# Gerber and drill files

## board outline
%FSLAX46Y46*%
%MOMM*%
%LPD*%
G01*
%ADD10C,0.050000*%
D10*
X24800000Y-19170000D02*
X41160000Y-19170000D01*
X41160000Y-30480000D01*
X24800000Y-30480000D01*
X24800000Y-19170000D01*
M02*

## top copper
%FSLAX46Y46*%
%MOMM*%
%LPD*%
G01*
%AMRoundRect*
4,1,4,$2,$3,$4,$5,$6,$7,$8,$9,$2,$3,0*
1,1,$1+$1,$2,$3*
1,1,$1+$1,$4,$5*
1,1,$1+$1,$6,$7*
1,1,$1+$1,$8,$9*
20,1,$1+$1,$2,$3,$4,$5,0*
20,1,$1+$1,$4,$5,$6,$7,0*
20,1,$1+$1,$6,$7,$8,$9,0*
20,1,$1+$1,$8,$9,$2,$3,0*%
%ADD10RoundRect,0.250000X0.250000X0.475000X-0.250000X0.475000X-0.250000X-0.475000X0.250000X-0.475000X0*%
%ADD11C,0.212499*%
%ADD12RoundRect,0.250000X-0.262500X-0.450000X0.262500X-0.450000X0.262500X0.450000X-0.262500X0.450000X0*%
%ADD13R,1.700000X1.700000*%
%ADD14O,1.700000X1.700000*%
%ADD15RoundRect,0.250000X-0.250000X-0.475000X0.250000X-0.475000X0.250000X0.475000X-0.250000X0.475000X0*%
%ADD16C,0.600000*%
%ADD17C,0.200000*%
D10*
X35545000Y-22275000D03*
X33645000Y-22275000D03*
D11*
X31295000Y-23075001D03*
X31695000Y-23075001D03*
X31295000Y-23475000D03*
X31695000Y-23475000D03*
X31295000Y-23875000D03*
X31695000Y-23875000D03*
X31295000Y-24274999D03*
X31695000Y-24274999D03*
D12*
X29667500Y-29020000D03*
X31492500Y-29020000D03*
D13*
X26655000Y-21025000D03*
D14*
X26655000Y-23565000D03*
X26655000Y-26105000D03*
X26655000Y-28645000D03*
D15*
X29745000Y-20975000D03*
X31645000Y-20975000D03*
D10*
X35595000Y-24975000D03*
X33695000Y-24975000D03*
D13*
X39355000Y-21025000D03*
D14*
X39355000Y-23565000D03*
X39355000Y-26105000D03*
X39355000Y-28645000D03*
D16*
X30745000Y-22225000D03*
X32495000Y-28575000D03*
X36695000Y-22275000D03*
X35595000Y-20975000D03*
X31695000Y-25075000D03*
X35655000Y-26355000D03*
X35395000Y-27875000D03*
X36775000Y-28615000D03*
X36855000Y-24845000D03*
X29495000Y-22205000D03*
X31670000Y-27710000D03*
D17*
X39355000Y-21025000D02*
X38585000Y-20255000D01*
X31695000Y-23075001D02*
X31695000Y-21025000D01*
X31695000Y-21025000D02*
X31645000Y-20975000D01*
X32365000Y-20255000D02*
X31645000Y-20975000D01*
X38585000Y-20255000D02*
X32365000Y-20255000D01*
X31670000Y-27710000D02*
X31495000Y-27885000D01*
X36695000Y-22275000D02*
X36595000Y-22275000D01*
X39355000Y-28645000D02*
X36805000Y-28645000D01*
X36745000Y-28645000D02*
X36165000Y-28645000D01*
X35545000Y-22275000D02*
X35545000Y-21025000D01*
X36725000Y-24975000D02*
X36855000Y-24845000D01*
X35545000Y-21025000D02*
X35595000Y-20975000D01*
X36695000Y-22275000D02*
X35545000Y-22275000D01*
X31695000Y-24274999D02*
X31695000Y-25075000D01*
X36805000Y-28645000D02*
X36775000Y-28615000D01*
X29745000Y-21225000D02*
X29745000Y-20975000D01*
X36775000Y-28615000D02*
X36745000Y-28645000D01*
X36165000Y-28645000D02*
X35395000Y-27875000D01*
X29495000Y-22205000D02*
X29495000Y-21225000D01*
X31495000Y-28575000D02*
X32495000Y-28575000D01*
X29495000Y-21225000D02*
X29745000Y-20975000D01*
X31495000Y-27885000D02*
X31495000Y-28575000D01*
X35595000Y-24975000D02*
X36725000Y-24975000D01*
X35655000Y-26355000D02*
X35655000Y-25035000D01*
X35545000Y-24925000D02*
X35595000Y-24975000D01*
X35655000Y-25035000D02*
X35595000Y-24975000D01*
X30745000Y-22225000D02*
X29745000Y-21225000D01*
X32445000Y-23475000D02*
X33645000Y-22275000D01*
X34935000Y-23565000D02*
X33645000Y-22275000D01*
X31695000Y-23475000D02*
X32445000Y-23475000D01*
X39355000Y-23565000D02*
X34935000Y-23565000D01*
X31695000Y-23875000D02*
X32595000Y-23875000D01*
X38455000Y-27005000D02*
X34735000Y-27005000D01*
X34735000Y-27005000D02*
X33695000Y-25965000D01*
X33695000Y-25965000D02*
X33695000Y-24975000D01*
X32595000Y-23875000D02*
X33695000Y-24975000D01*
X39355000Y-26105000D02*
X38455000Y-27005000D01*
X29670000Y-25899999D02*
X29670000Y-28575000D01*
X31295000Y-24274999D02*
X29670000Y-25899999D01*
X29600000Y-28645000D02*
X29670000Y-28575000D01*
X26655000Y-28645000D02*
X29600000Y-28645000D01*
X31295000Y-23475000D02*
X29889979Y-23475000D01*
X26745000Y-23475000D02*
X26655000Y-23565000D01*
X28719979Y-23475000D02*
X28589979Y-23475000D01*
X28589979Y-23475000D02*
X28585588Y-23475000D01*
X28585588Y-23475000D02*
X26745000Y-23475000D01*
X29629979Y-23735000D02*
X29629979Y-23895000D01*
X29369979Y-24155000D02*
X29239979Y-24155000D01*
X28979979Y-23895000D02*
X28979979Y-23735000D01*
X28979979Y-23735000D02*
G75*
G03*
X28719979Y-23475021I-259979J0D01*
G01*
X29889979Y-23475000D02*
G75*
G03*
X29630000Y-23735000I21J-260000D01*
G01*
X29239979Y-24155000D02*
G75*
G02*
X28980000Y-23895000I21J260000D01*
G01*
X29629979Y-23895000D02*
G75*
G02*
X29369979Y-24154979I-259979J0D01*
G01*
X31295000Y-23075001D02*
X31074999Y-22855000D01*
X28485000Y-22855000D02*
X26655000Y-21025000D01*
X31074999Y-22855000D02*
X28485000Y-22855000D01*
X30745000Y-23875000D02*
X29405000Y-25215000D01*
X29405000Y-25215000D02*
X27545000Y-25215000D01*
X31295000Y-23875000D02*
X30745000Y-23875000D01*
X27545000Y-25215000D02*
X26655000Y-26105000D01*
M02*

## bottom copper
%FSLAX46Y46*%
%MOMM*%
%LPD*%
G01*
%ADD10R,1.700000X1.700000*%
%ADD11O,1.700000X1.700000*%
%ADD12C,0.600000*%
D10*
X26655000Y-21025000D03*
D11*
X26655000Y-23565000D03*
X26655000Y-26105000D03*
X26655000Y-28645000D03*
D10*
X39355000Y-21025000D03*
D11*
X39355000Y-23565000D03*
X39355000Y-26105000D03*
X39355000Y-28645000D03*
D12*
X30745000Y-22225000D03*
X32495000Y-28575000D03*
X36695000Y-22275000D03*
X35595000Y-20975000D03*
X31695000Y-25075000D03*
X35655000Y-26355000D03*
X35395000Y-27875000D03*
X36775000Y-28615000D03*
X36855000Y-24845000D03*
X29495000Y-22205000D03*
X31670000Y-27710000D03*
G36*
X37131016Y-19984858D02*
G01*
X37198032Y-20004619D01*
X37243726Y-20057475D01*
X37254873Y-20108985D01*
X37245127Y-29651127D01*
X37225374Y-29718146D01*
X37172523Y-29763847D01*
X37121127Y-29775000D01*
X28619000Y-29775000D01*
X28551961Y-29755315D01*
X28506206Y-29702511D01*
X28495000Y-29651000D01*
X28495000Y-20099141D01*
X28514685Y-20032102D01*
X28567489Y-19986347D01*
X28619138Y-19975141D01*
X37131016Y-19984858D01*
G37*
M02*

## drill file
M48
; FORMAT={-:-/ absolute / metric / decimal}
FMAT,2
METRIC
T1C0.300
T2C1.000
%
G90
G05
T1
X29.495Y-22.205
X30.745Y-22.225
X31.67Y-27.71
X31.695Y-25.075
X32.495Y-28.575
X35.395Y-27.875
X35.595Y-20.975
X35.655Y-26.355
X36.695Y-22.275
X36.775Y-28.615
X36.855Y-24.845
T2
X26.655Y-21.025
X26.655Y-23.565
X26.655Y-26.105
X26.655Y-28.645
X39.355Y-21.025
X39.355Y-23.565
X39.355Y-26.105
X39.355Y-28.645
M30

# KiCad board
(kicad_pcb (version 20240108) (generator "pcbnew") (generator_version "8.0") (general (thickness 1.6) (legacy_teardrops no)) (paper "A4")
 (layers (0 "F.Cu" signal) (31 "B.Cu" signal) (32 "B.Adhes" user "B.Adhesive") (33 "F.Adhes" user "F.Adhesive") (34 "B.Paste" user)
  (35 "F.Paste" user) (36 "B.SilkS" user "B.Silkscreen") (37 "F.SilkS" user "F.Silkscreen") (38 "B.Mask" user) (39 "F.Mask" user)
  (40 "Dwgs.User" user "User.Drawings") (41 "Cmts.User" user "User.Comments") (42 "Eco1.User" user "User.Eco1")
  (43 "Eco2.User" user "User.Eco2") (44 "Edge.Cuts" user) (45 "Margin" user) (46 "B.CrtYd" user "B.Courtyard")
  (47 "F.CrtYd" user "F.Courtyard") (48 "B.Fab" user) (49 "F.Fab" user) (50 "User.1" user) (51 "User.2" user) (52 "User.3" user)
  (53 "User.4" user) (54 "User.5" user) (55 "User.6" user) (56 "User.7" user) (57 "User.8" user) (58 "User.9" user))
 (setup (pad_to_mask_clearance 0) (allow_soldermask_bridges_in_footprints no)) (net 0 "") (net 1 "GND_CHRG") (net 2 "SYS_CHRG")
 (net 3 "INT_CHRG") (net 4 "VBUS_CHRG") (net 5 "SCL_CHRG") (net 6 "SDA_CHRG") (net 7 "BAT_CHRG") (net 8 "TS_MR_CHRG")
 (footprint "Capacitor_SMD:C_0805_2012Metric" (layer "F.Cu") (at 34.595 22.275 180)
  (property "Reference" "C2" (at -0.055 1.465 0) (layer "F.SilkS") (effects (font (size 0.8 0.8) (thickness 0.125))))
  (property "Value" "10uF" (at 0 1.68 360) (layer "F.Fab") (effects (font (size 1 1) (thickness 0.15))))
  (pad "1" smd roundrect (at -0.95 0 180) (size 1 1.45) (layers "F.Cu" "F.Paste" "F.Mask") (roundrect_rratio 0.25) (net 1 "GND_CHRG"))
  (pad "2" smd roundrect (at 0.95 0 180) (size 1 1.45) (layers "F.Cu" "F.Paste" "F.Mask") (roundrect_rratio 0.25) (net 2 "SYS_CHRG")))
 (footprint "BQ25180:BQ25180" (layer "F.Cu") (at 31.495 23.675)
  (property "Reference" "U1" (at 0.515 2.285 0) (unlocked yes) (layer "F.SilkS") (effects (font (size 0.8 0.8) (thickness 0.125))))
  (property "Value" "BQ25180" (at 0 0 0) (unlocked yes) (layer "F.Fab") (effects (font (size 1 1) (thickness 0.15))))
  (pad "1" smd circle (at -0.2 -0.599999) (size 0.212499 0.212499) (layers "F.Cu" "F.Paste" "F.Mask") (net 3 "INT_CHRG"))
  (pad "2" smd circle (at 0.2 -0.599999) (size 0.212499 0.212499) (layers "F.Cu" "F.Paste" "F.Mask") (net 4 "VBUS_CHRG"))
  (pad "3" smd circle (at -0.2 -0.2) (size 0.212499 0.212499) (layers "F.Cu" "F.Paste" "F.Mask") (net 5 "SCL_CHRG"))
  (pad "4" smd circle (at 0.2 -0.2) (size 0.212499 0.212499) (layers "F.Cu" "F.Paste" "F.Mask") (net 2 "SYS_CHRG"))
  (pad "5" smd circle (at -0.2 0.2) (size 0.212499 0.212499) (layers "F.Cu" "F.Paste" "F.Mask") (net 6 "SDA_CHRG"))
  (pad "6" smd circle (at 0.2 0.2) (size 0.212499 0.212499) (layers "F.Cu" "F.Paste" "F.Mask") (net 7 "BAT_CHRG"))
  (pad "7" smd circle (at -0.2 0.599999) (size 0.212499 0.212499) (layers "F.Cu" "F.Paste" "F.Mask") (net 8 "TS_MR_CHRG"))
  (pad "8" smd circle (at 0.2 0.599999) (size 0.212499 0.212499) (layers "F.Cu" "F.Paste" "F.Mask") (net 1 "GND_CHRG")))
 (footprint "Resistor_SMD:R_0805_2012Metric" (layer "F.Cu") (at 30.58 29.02)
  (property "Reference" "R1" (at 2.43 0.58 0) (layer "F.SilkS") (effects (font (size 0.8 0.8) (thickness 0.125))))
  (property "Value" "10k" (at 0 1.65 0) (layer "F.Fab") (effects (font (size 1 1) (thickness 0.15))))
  (pad "1" smd roundrect (at -0.9125 0) (size 1.025 1.4) (layers "F.Cu" "F.Paste" "F.Mask") (roundrect_rratio 0.243902) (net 8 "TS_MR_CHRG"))
  (pad "2" smd roundrect (at 0.9125 0) (size 1.025 1.4) (layers "F.Cu" "F.Paste" "F.Mask") (roundrect_rratio 0.243902) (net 1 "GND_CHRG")))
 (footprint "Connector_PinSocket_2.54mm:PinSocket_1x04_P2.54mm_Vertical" (layer "F.Cu") (at 26.655 21.025)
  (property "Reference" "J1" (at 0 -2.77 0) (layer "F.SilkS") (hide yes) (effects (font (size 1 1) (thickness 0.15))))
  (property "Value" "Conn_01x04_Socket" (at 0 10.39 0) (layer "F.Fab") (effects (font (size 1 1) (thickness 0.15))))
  (pad "1" thru_hole rect (at 0 0) (size 1.7 1.7) (drill 1) (layers "*.Cu" "*.Mask") (remove_unused_layers no) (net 3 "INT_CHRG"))
  (pad "2" thru_hole oval (at 0 2.54) (size 1.7 1.7) (drill 1) (layers "*.Cu" "*.Mask") (remove_unused_layers no) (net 5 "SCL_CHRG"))
  (pad "3" thru_hole oval (at 0 5.08) (size 1.7 1.7) (drill 1) (layers "*.Cu" "*.Mask") (remove_unused_layers no) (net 6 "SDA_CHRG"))
  (pad "4" thru_hole oval (at 0 7.62) (size 1.7 1.7) (drill 1) (layers "*.Cu" "*.Mask") (remove_unused_layers no) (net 8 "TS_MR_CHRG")))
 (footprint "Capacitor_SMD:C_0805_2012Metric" (layer "F.Cu") (at 30.695 20.975)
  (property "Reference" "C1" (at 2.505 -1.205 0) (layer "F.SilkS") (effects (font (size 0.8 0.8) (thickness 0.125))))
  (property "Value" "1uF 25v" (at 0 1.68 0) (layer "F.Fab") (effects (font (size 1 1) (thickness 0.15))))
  (pad "1" smd roundrect (at -0.95 0) (size 1 1.45) (layers "F.Cu" "F.Paste" "F.Mask") (roundrect_rratio 0.25) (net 1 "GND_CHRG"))
  (pad "2" smd roundrect (at 0.95 0) (size 1 1.45) (layers "F.Cu" "F.Paste" "F.Mask") (roundrect_rratio 0.25) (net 4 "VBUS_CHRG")))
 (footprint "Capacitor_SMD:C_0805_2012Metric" (layer "F.Cu") (at 34.645 24.975 180)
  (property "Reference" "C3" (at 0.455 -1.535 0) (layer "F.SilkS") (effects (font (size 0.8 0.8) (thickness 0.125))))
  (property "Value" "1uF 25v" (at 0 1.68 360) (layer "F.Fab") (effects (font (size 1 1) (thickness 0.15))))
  (pad "1" smd roundrect (at -0.95 0 180) (size 1 1.45) (layers "F.Cu" "F.Paste" "F.Mask") (roundrect_rratio 0.25) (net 1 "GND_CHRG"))
  (pad "2" smd roundrect (at 0.95 0 180) (size 1 1.45) (layers "F.Cu" "F.Paste" "F.Mask") (roundrect_rratio 0.25) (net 7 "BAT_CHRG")))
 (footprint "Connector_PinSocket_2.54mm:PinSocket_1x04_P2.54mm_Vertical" (layer "F.Cu") (at 39.355 21.025)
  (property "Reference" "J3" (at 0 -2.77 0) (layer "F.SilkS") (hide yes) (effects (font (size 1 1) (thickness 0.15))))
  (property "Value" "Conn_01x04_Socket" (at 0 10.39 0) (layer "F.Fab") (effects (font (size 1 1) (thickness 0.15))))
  (pad "1" thru_hole rect (at 0 0) (size 1.7 1.7) (drill 1) (layers "*.Cu" "*.Mask") (remove_unused_layers no) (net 4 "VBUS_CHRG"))
  (pad "2" thru_hole oval (at 0 2.54) (size 1.7 1.7) (drill 1) (layers "*.Cu" "*.Mask") (remove_unused_layers no) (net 2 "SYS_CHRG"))
  (pad "3" thru_hole oval (at 0 5.08) (size 1.7 1.7) (drill 1) (layers "*.Cu" "*.Mask") (remove_unused_layers no) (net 7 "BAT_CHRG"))
  (pad "4" thru_hole oval (at 0 7.62) (size 1.7 1.7) (drill 1) (layers "*.Cu" "*.Mask") (remove_unused_layers no) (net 1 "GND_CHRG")))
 (gr_rect (start 24.8 19.17) (end 41.16 30.48) (stroke (width 0.05) (type default)) (fill none) (layer "Edge.Cuts"))
 (segment (start 39.355 21.025) (end 38.585 20.255) (width 0.2) (layer "F.Cu") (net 4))
 (segment (start 31.695 23.075001) (end 31.695 21.025) (width 0.2) (layer "F.Cu") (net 4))
 (segment (start 31.695 21.025) (end 31.645 20.975) (width 0.2) (layer "F.Cu") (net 4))
 (segment (start 32.365 20.255) (end 31.645 20.975) (width 0.2) (layer "F.Cu") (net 4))
 (segment (start 38.585 20.255) (end 32.365 20.255) (width 0.2) (layer "F.Cu") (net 4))
 (segment (start 31.67 27.71) (end 31.495 27.885) (width 0.2) (layer "F.Cu") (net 1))
 (segment (start 36.695 22.275) (end 36.595 22.275) (width 0.2) (layer "F.Cu") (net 1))
 (segment (start 39.355 28.645) (end 36.805 28.645) (width 0.2) (layer "F.Cu") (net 1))
 (segment (start 36.745 28.645) (end 36.165 28.645) (width 0.2) (layer "F.Cu") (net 1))
 (segment (start 35.545 22.275) (end 35.545 21.025) (width 0.2) (layer "F.Cu") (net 1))
 (segment (start 36.725 24.975) (end 36.855 24.845) (width 0.2) (layer "F.Cu") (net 1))
 (segment (start 35.545 21.025) (end 35.595 20.975) (width 0.2) (layer "F.Cu") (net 1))
 (segment (start 36.695 22.275) (end 35.545 22.275) (width 0.2) (layer "F.Cu") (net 1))
 (segment (start 31.695 24.274999) (end 31.695 25.075) (width 0.2) (layer "F.Cu") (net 1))
 (segment (start 36.805 28.645) (end 36.775 28.615) (width 0.2) (layer "F.Cu") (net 1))
 (segment (start 29.745 21.225) (end 29.745 20.975) (width 0.2) (layer "F.Cu") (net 1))
 (segment (start 36.775 28.615) (end 36.745 28.645) (width 0.2) (layer "F.Cu") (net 1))
 (segment (start 36.165 28.645) (end 35.395 27.875) (width 0.2) (layer "F.Cu") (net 1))
 (segment (start 29.495 22.205) (end 29.495 21.225) (width 0.2) (layer "F.Cu") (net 1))
 (segment (start 31.495 28.575) (end 32.495 28.575) (width 0.2) (layer "F.Cu") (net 1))
 (segment (start 29.495 21.225) (end 29.745 20.975) (width 0.2) (layer "F.Cu") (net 1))
 (segment (start 31.495 27.885) (end 31.495 28.575) (width 0.2) (layer "F.Cu") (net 1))
 (segment (start 35.595 24.975) (end 36.725 24.975) (width 0.2) (layer "F.Cu") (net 1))
 (segment (start 35.655 26.355) (end 35.655 25.035) (width 0.2) (layer "F.Cu") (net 1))
 (segment (start 35.545 24.925) (end 35.595 24.975) (width 0.2) (layer "F.Cu") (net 1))
 (segment (start 35.655 25.035) (end 35.595 24.975) (width 0.2) (layer "F.Cu") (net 1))
 (segment (start 30.745 22.225) (end 29.745 21.225) (width 0.2) (layer "F.Cu") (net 1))
 (via (at 30.745 22.225) (size 0.6) (drill 0.3) (layers "F.Cu" "B.Cu") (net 1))
 (via (at 32.495 28.575) (size 0.6) (drill 0.3) (layers "F.Cu" "B.Cu") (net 1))
 (via (at 36.695 22.275) (size 0.6) (drill 0.3) (layers "F.Cu" "B.Cu") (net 1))
 (via (at 35.595 20.975) (size 0.6) (drill 0.3) (layers "F.Cu" "B.Cu") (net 1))
 (via (at 31.695 25.075) (size 0.6) (drill 0.3) (layers "F.Cu" "B.Cu") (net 1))
 (via (at 35.655 26.355) (size 0.6) (drill 0.3) (layers "F.Cu" "B.Cu") (free yes) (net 1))
 (via (at 35.395 27.875) (size 0.6) (drill 0.3) (layers "F.Cu" "B.Cu") (free yes) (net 1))
 (via (at 36.775 28.615) (size 0.6) (drill 0.3) (layers "F.Cu" "B.Cu") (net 1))
 (via (at 36.855 24.845) (size 0.6) (drill 0.3) (layers "F.Cu" "B.Cu") (free yes) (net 1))
 (via (at 29.495 22.205) (size 0.6) (drill 0.3) (layers "F.Cu" "B.Cu") (free yes) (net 1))
 (via (at 31.67 27.71) (size 0.6) (drill 0.3) (layers "F.Cu" "B.Cu") (free yes) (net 1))
 (segment (start 32.445 23.475) (end 33.645 22.275) (width 0.2) (layer "F.Cu") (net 2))
 (segment (start 34.935 23.565) (end 33.645 22.275) (width 0.2) (layer "F.Cu") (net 2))
 (segment (start 31.695 23.475) (end 32.445 23.475) (width 0.2) (layer "F.Cu") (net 2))
 (segment (start 39.355 23.565) (end 34.935 23.565) (width 0.2) (layer "F.Cu") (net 2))
 (segment (start 31.695 23.875) (end 32.595 23.875) (width 0.2) (layer "F.Cu") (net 7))
 (segment (start 38.455 27.005) (end 34.735 27.005) (width 0.2) (layer "F.Cu") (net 7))
 (segment (start 34.735 27.005) (end 33.695 25.965) (width 0.2) (layer "F.Cu") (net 7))
 (segment (start 33.695 25.965) (end 33.695 24.975) (width 0.2) (layer "F.Cu") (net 7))
 (segment (start 32.595 23.875) (end 33.695 24.975) (width 0.2) (layer "F.Cu") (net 7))
 (segment (start 39.355 26.105) (end 38.455 27.005) (width 0.2) (layer "F.Cu") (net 7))
 (segment (start 29.67 25.899999) (end 29.67 28.575) (width 0.2) (layer "F.Cu") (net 8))
 (segment (start 31.295 24.274999) (end 29.67 25.899999) (width 0.2) (layer "F.Cu") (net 8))
 (segment (start 29.6 28.645) (end 29.67 28.575) (width 0.2) (layer "F.Cu") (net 8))
 (segment (start 26.655 28.645) (end 29.6 28.645) (width 0.2) (layer "F.Cu") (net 8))
 (segment (start 31.295 23.475) (end 29.889979 23.475) (width 0.2) (layer "F.Cu") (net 5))
 (segment (start 26.745 23.475) (end 26.655 23.565) (width 0.2) (layer "F.Cu") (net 5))
 (segment (start 28.719979 23.475) (end 28.589979 23.475) (width 0.2) (layer "F.Cu") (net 5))
 (segment (start 28.589979 23.475) (end 28.585588 23.475) (width 0.2) (layer "F.Cu") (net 5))
 (segment (start 28.585588 23.475) (end 26.745 23.475) (width 0.2) (layer "F.Cu") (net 5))
 (segment (start 29.629979 23.735) (end 29.629979 23.895) (width 0.2) (layer "F.Cu") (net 5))
 (segment (start 29.369979 24.155) (end 29.239979 24.155) (width 0.2) (layer "F.Cu") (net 5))
 (segment (start 28.979979 23.895) (end 28.979979 23.735) (width 0.2) (layer "F.Cu") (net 5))
 (arc (start 28.979979 23.735) (mid 28.903827 23.551152) (end 28.719979 23.475) (width 0.2) (layer "F.Cu") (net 5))
 (arc (start 29.889979 23.475) (mid 29.706131 23.551152) (end 29.629979 23.735) (width 0.2) (layer "F.Cu") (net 5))
 (arc (start 29.239979 24.155) (mid 29.056131 24.078848) (end 28.979979 23.895) (width 0.2) (layer "F.Cu") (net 5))
 (arc (start 29.629979 23.895) (mid 29.553827 24.078848) (end 29.369979 24.155) (width 0.2) (layer "F.Cu") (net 5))
 (segment (start 31.295 23.075001) (end 31.074999 22.855) (width 0.2) (layer "F.Cu") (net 3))
 (segment (start 28.485 22.855) (end 26.655 21.025) (width 0.2) (layer "F.Cu") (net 3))
 (segment (start 31.074999 22.855) (end 28.485 22.855) (width 0.2) (layer "F.Cu") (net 3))
 (segment (start 30.745 23.875) (end 29.405 25.215) (width 0.2) (layer "F.Cu") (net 6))
 (segment (start 29.405 25.215) (end 27.545 25.215) (width 0.2) (layer "F.Cu") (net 6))
 (segment (start 31.295 23.875) (end 30.745 23.875) (width 0.2) (layer "F.Cu") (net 6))
 (segment (start 27.545 25.215) (end 26.655 26.105) (width 0.2) (layer "F.Cu") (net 6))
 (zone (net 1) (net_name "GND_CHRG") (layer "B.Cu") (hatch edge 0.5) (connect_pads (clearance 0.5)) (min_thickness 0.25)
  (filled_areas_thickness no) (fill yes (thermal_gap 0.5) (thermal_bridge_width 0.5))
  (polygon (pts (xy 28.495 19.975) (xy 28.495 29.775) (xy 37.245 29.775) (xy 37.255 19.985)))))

